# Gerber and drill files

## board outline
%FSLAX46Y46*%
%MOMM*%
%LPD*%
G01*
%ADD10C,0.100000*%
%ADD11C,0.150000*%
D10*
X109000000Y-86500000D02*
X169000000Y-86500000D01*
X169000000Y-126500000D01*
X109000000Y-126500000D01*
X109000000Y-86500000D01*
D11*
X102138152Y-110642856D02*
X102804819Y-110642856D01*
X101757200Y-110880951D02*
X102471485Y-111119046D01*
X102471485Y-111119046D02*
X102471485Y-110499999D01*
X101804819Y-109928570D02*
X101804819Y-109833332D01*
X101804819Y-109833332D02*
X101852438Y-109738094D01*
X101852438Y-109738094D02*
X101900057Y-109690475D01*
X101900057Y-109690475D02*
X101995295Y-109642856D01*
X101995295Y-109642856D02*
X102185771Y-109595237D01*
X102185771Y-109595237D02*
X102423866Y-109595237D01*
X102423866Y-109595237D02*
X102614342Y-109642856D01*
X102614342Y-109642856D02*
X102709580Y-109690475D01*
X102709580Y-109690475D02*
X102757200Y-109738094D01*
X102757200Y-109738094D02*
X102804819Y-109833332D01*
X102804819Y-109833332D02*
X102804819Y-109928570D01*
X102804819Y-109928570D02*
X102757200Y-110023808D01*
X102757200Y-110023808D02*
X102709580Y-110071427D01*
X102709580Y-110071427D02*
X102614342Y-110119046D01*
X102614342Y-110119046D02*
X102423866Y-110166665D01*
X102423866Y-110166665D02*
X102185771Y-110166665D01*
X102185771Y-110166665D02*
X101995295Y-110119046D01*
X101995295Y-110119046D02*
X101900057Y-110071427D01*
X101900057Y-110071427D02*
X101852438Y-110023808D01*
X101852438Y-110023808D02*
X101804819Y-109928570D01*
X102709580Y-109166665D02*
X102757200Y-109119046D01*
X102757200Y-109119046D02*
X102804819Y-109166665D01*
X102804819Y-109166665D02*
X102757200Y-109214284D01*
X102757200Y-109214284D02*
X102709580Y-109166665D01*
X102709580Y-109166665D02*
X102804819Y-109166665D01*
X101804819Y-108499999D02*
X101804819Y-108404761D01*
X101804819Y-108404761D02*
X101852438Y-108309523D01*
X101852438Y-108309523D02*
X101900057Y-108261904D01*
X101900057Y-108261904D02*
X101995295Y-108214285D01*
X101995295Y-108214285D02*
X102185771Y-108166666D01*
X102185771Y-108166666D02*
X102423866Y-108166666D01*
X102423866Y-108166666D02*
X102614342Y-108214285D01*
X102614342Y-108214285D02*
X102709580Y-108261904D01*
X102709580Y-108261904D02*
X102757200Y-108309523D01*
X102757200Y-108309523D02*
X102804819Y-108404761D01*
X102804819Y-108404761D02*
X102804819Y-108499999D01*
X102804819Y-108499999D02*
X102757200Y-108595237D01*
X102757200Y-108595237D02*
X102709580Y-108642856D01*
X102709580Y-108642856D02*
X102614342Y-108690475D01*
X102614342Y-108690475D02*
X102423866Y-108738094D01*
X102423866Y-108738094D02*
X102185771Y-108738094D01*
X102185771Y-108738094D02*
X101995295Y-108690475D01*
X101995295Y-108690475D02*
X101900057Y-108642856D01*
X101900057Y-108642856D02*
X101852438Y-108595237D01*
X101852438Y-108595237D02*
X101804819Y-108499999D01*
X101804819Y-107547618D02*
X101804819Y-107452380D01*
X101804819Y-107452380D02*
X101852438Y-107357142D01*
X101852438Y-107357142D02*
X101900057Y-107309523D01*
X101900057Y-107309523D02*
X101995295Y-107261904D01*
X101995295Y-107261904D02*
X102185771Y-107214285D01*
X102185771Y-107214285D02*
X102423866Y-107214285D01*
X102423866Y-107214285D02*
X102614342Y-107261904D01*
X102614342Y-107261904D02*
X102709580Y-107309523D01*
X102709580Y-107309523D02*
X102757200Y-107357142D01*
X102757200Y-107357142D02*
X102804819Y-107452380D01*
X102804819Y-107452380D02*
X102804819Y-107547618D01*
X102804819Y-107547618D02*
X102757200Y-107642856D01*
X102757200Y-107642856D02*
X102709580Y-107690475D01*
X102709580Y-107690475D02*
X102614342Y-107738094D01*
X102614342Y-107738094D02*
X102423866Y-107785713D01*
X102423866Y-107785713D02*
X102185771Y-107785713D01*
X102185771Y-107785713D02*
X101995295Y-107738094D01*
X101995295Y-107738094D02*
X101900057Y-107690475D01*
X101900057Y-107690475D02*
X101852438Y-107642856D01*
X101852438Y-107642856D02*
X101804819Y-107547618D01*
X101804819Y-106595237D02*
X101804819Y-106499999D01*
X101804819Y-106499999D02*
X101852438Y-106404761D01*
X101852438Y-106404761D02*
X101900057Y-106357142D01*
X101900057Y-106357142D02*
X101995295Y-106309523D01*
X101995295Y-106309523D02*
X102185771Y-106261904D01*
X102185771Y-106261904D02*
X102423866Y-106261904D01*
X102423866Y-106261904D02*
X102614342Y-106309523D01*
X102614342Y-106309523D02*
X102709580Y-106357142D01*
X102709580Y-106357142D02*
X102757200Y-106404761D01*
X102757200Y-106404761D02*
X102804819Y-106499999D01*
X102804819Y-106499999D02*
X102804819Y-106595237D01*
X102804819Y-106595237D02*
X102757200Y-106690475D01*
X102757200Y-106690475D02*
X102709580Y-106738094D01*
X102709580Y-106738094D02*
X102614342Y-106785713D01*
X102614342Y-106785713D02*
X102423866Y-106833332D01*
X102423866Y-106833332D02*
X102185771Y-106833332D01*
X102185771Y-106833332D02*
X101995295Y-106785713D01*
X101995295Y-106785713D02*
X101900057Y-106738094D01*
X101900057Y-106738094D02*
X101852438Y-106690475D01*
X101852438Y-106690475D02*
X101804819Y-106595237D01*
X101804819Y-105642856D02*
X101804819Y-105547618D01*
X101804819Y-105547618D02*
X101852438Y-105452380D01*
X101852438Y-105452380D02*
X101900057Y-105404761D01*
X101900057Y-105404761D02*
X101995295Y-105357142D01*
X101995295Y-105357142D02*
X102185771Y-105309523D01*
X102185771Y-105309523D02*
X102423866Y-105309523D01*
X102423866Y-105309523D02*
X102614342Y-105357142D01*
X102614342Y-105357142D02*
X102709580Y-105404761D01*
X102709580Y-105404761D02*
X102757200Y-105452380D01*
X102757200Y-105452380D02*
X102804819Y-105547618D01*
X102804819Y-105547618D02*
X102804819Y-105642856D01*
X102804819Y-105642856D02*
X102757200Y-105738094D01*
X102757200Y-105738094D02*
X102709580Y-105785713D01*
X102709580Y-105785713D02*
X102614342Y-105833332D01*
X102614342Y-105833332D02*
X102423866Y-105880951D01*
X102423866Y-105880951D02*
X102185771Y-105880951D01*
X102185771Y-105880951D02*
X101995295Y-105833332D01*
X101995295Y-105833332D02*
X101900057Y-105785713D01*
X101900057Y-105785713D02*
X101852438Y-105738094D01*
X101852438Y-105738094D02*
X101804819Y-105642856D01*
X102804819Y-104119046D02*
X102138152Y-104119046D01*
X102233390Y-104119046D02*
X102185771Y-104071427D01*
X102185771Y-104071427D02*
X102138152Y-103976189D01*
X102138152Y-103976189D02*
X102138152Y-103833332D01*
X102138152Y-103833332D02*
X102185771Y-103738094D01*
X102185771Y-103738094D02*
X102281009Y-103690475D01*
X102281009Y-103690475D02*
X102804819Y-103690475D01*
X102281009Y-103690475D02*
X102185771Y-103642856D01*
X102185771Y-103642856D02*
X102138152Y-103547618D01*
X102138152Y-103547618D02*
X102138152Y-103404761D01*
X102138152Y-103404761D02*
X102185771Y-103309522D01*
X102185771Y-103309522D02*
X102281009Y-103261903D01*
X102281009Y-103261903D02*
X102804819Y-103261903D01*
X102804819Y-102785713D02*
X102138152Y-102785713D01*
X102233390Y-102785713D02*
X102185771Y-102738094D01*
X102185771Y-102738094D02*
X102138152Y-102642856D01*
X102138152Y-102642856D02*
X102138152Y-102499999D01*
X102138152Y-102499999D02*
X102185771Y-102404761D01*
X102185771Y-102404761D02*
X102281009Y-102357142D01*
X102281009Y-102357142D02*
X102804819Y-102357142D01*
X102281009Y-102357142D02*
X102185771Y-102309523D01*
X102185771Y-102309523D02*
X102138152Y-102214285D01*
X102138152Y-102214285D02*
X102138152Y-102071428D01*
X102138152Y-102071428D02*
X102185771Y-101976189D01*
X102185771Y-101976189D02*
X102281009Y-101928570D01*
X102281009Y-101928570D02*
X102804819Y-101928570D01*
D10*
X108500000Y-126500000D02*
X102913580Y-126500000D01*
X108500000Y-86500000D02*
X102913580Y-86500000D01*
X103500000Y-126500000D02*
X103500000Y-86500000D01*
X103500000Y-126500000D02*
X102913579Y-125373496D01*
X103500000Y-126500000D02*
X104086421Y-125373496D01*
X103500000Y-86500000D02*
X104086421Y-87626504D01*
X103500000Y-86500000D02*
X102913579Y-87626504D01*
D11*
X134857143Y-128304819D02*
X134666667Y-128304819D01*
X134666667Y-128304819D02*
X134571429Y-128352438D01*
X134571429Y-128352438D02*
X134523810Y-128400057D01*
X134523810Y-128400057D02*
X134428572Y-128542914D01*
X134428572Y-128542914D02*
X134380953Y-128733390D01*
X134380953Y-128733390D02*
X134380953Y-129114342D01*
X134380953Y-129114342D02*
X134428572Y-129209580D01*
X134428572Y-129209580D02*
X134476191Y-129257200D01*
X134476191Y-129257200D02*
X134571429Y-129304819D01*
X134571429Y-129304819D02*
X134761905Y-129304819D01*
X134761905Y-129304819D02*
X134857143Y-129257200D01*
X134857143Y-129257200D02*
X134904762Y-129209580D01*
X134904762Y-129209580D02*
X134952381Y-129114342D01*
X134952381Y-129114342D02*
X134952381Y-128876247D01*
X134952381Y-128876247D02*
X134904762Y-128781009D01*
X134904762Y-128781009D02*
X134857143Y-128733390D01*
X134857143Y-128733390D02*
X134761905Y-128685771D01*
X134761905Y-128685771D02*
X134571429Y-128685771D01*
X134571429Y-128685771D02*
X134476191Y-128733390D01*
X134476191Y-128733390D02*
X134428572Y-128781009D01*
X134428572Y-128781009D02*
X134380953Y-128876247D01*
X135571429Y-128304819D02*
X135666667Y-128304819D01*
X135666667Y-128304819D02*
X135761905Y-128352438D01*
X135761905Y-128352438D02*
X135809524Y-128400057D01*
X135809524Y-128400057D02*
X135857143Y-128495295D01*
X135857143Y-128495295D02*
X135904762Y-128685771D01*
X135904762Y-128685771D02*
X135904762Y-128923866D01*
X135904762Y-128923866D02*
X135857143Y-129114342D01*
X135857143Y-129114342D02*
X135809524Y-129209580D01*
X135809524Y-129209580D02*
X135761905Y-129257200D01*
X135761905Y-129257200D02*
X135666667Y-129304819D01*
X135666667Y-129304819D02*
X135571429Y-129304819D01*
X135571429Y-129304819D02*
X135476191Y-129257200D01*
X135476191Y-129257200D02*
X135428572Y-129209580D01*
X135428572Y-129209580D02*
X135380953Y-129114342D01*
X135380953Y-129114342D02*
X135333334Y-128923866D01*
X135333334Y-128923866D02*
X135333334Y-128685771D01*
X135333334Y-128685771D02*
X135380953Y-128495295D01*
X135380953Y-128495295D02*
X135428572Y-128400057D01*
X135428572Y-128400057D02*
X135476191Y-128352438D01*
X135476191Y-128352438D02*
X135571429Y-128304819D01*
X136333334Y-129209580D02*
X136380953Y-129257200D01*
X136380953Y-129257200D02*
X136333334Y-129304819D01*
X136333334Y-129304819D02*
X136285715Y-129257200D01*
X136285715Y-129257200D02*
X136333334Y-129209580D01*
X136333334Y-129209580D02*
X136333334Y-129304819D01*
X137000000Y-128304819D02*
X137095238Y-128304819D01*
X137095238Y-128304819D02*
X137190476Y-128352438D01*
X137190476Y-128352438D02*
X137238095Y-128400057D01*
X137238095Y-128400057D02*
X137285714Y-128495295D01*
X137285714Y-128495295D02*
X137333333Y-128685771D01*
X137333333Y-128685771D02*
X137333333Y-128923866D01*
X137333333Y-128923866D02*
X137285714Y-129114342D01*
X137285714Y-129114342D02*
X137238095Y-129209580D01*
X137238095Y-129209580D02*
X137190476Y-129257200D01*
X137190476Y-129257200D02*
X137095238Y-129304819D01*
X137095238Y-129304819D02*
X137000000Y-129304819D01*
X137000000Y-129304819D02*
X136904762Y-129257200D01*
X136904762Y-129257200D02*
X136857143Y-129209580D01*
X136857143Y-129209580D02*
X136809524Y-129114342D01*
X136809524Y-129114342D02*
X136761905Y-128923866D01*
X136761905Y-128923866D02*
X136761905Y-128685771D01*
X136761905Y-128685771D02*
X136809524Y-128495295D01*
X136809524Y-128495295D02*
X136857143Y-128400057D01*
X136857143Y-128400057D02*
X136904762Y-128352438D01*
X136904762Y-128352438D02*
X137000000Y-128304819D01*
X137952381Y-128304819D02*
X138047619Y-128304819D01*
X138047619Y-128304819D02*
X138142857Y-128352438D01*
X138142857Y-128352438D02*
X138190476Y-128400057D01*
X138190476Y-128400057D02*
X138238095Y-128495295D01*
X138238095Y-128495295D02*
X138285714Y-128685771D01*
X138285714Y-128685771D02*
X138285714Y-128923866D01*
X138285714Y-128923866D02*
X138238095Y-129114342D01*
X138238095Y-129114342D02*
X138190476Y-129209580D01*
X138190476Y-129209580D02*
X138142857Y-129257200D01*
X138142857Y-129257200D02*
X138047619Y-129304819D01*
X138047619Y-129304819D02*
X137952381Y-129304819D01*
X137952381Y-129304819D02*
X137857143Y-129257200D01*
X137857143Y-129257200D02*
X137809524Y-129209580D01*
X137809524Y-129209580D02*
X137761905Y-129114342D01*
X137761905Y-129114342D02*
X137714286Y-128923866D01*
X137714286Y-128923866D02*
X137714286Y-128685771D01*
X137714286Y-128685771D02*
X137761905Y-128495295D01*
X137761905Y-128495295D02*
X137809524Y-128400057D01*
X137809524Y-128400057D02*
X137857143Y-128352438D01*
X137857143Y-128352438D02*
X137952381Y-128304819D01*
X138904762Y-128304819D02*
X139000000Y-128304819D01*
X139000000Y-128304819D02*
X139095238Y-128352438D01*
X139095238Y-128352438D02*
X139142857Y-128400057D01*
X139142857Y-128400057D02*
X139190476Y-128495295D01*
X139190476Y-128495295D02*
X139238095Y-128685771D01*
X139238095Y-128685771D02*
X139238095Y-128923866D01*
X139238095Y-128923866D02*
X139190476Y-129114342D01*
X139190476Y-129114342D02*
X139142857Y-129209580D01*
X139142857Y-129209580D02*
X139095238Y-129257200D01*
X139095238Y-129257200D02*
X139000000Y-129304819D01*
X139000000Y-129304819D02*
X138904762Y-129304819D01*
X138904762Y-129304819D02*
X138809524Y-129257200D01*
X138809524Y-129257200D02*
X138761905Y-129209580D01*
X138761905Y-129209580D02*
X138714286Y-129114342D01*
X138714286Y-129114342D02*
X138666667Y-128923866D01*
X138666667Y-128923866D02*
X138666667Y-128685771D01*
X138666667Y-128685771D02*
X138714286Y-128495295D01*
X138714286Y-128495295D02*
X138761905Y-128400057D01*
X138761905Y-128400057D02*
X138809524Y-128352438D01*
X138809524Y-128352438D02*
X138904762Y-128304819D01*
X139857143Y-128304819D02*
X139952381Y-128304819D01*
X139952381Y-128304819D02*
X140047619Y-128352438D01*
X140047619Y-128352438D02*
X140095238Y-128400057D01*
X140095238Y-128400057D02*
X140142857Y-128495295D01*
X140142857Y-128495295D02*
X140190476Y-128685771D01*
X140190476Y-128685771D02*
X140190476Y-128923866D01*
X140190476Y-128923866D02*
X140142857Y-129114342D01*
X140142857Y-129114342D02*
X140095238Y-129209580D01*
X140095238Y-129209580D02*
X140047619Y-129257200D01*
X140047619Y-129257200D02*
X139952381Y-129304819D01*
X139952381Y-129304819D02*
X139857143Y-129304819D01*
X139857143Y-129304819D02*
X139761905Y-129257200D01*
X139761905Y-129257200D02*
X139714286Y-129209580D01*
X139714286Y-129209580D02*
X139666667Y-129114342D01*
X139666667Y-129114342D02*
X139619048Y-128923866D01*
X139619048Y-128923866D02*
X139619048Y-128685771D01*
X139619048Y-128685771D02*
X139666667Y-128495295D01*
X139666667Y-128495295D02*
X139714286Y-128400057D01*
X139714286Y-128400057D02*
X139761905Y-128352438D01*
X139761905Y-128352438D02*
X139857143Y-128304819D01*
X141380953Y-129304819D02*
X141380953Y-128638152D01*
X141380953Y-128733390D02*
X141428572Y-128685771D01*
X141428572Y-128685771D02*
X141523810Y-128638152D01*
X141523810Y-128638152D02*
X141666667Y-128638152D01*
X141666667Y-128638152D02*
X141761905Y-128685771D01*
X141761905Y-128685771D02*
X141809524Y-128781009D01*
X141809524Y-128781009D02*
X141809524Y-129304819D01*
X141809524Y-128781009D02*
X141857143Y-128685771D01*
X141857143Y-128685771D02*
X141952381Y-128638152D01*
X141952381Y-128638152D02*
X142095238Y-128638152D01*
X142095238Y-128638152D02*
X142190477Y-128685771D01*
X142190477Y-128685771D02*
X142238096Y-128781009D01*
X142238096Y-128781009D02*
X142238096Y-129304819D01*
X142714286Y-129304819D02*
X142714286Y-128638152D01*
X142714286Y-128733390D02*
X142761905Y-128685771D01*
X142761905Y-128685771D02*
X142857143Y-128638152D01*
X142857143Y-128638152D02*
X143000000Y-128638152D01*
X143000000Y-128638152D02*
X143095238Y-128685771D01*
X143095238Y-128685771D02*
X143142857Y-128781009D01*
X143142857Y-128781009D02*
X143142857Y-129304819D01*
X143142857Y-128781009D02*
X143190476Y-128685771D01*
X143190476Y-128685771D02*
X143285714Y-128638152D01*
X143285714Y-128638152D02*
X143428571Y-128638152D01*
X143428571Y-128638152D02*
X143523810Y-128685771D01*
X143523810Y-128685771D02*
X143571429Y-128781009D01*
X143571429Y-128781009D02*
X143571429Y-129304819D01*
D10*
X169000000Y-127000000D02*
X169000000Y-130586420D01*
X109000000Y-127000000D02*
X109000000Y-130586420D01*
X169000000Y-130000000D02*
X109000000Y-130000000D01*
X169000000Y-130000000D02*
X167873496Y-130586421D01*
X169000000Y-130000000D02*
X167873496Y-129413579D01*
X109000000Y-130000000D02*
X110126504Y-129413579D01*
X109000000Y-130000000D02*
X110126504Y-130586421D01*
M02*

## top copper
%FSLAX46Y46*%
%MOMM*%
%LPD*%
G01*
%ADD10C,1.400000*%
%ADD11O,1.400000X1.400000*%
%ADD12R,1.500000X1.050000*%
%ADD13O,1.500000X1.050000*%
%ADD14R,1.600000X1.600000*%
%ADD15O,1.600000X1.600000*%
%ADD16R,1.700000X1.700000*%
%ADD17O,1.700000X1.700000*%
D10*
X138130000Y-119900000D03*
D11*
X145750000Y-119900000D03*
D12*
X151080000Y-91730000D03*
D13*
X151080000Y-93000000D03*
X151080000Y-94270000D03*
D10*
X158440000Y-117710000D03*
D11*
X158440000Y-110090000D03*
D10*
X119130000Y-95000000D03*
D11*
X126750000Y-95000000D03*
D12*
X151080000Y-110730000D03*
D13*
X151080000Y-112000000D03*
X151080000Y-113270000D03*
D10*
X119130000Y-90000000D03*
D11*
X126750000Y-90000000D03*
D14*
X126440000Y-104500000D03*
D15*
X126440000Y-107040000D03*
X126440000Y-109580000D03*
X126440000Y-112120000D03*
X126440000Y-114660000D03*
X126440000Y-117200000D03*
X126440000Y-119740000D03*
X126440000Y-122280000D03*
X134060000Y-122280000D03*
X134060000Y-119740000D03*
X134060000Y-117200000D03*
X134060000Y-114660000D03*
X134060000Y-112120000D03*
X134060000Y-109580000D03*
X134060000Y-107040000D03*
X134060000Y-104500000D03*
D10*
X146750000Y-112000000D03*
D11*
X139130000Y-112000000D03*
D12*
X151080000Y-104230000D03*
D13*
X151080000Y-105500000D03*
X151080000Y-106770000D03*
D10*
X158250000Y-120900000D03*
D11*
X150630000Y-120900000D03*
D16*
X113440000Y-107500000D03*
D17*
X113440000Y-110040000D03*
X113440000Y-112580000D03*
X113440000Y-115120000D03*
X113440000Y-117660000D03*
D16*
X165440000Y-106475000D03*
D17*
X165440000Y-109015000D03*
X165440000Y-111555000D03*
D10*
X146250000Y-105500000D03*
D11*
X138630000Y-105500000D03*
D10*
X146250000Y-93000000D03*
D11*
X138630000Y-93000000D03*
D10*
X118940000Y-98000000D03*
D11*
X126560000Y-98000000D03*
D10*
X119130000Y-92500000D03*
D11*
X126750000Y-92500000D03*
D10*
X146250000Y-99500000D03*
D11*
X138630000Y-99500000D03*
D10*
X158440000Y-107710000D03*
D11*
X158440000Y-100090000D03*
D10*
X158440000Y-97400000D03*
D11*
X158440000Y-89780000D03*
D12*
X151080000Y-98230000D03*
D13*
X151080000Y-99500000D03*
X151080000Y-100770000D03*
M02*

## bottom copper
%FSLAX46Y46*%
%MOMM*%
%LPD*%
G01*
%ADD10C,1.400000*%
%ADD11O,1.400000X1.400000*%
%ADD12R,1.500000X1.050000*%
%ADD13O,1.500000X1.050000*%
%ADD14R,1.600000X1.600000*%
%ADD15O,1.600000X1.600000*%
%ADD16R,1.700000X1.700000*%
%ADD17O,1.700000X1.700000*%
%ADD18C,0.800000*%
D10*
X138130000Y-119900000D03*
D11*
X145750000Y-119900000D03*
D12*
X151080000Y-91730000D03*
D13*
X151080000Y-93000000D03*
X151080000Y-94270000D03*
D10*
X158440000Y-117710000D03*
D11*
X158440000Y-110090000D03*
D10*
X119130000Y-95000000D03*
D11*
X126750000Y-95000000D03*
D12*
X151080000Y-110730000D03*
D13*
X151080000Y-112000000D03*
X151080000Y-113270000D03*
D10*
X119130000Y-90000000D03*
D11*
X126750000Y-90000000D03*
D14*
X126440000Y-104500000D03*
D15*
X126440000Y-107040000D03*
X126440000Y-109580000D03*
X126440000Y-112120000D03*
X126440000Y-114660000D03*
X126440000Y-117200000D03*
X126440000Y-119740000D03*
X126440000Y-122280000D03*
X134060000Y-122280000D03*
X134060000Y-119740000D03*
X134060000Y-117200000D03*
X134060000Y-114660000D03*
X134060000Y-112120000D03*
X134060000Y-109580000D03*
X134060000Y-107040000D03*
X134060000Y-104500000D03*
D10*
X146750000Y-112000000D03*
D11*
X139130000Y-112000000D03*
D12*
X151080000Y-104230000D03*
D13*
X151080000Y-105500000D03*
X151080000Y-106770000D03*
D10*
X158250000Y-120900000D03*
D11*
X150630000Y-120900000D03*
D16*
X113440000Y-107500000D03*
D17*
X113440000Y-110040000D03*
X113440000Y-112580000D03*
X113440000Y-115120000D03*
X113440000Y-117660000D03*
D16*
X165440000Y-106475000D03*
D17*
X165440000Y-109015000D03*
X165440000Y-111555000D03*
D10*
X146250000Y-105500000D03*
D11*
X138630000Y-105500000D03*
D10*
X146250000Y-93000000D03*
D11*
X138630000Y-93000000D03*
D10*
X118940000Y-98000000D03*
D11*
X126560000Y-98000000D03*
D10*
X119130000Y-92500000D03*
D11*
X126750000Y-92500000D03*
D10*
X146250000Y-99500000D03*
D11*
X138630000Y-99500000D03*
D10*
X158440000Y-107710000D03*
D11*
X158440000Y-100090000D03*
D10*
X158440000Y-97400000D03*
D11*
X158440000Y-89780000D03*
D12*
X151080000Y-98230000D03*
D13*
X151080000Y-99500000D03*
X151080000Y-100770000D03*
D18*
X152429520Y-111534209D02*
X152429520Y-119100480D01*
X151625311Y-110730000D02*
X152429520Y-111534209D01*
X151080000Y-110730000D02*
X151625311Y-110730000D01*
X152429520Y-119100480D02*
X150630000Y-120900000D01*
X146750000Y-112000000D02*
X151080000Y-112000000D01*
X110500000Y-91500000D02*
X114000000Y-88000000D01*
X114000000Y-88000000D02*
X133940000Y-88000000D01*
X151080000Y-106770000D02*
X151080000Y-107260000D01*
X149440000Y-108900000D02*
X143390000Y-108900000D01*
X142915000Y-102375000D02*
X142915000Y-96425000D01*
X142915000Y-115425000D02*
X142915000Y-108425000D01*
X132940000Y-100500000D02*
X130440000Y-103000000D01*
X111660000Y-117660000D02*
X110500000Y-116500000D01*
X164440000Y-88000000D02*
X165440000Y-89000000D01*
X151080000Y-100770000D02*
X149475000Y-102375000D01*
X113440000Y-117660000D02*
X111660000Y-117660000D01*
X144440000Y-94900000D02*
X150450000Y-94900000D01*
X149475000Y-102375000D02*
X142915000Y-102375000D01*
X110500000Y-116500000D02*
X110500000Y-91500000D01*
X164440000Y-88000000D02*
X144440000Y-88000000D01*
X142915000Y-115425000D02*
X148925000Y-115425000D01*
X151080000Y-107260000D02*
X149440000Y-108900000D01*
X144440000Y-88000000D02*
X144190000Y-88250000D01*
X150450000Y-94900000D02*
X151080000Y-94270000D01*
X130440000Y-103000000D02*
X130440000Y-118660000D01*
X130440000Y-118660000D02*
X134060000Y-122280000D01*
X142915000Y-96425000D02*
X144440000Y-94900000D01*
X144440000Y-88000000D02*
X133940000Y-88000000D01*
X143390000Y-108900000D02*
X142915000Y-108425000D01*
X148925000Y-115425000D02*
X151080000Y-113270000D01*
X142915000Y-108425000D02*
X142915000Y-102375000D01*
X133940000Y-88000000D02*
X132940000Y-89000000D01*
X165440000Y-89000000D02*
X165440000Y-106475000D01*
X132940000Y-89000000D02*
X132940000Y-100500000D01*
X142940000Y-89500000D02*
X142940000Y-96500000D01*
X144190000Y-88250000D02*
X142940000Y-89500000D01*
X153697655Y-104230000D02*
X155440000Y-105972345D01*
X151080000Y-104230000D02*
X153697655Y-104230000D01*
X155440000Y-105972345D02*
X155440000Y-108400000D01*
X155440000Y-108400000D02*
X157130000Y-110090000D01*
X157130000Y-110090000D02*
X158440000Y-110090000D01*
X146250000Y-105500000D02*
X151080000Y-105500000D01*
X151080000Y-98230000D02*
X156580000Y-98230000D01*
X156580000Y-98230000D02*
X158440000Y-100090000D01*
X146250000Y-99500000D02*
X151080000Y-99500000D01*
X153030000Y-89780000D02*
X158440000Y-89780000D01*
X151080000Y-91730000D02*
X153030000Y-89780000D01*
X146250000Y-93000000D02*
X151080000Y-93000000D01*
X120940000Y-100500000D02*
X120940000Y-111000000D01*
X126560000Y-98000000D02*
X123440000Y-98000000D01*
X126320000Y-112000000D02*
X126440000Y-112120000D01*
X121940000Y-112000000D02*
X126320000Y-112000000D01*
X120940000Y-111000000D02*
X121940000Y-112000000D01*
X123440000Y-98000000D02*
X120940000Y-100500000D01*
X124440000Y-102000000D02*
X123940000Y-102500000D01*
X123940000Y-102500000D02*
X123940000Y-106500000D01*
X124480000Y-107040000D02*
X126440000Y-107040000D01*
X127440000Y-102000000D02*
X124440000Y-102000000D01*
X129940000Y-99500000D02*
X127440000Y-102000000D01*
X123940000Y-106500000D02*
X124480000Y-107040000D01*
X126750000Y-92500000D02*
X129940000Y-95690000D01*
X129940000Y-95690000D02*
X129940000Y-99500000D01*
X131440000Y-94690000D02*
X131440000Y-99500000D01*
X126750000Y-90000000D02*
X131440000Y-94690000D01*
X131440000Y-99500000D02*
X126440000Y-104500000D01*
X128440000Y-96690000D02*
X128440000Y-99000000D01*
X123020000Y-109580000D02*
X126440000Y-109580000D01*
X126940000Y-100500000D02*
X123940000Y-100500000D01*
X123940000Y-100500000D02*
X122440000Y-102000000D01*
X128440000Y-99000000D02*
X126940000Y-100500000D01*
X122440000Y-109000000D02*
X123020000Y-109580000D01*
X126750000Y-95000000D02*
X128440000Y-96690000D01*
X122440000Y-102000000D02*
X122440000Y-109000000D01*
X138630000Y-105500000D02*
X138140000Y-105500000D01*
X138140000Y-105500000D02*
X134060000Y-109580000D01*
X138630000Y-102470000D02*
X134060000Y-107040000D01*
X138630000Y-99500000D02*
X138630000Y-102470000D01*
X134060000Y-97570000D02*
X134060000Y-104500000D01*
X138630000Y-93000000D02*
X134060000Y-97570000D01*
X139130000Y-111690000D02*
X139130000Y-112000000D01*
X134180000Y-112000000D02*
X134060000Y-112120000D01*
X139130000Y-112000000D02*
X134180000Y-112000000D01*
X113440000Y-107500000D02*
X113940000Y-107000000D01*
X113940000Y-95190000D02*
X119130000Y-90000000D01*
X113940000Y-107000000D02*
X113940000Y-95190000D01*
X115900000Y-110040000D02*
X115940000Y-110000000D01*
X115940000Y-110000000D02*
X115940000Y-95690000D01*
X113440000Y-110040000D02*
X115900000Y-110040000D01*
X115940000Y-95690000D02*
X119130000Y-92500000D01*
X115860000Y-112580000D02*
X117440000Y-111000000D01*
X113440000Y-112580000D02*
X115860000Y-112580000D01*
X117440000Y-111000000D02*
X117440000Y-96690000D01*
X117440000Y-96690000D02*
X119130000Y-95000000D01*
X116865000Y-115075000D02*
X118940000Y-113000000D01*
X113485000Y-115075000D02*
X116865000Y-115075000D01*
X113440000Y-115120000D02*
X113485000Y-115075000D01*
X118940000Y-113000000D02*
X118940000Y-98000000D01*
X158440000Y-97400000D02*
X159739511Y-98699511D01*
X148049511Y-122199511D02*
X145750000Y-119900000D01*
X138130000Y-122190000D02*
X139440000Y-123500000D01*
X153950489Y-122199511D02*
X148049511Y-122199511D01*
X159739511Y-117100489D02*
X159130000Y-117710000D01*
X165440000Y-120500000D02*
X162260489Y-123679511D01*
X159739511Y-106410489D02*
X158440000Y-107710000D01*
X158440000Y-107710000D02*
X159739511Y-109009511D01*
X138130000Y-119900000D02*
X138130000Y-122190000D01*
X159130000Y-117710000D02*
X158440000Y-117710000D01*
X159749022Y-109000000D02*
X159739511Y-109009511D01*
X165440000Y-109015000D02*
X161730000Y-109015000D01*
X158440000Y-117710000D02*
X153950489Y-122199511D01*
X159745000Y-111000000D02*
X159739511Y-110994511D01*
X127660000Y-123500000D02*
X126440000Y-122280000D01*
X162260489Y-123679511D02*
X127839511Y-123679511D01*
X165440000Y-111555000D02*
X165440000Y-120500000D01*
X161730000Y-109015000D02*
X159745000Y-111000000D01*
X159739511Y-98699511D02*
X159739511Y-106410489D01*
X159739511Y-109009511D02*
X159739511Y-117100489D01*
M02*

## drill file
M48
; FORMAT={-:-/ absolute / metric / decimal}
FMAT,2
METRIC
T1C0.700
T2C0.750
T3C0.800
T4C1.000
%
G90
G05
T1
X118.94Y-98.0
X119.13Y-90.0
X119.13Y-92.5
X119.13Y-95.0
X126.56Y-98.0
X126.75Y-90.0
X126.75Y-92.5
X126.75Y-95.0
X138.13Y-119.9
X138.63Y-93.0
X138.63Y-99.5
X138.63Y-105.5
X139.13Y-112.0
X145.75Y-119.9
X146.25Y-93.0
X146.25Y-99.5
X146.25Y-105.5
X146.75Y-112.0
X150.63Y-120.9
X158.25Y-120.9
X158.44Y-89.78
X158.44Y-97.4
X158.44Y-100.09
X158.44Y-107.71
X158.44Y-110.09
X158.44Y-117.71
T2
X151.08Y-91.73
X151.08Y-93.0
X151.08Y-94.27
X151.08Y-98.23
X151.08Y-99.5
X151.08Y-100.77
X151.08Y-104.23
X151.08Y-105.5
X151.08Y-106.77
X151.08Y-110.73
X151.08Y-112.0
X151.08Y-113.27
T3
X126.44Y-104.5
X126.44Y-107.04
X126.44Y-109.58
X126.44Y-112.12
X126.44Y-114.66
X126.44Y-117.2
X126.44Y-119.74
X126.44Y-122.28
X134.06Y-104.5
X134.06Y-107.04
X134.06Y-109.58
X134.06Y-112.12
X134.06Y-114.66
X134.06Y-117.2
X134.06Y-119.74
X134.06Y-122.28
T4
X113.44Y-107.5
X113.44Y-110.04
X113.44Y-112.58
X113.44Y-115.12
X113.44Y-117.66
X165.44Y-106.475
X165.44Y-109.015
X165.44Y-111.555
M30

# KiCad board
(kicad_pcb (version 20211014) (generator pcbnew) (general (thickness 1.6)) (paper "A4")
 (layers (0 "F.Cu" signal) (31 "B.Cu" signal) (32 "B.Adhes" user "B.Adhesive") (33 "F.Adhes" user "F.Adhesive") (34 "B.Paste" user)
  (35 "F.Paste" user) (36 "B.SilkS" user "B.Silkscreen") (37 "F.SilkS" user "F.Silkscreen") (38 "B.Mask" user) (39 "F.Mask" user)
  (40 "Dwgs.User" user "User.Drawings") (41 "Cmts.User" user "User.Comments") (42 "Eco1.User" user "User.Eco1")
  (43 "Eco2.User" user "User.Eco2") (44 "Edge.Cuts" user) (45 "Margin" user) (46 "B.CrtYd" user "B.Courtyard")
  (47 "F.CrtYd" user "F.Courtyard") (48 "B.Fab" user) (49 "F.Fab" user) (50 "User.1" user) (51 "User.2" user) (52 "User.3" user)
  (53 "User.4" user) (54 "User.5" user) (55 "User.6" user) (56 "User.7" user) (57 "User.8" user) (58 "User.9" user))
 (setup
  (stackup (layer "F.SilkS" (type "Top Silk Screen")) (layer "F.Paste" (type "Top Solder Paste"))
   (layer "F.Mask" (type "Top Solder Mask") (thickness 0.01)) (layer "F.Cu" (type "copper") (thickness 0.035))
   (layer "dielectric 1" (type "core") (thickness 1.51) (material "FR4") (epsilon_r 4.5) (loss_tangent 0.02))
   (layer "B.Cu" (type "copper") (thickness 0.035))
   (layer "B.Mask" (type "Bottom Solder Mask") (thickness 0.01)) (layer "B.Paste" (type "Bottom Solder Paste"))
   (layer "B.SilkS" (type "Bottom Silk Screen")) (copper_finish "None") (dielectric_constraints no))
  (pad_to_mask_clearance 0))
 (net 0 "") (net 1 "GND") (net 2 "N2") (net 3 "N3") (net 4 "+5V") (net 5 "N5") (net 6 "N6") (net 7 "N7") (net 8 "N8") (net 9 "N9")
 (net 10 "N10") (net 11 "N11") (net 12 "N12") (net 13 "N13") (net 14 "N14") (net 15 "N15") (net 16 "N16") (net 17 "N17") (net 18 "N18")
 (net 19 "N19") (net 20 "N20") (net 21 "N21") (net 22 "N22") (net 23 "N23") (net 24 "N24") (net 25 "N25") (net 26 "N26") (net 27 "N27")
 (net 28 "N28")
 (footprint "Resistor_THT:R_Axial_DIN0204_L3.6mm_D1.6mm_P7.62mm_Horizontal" (layer "F.Cu") (at 138.13 119.9)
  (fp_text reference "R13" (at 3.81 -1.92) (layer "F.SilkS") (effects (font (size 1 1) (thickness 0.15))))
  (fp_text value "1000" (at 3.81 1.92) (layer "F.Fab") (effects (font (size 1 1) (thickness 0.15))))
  (pad "1" thru_hole circle (at 0 0) (size 1.4 1.4) (drill 0.7) (layers *.Cu *.Mask) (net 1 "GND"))
  (pad "2" thru_hole oval (at 7.62 0) (size 1.4 1.4) (drill 0.7) (layers *.Cu *.Mask) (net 1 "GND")))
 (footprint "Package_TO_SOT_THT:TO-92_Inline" (layer "F.Cu") (at 151.08 91.73 -90)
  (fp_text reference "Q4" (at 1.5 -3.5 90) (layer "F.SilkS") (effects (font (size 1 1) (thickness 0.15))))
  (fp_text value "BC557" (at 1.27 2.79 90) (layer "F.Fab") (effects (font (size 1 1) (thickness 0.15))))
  (pad "1" thru_hole rect (at 0 0 270) (size 1.05 1.5) (drill 0.75) (layers *.Cu *.Mask) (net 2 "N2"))
  (pad "2" thru_hole oval (at 1.27 0 270) (size 1.05 1.5) (drill 0.75) (layers *.Cu *.Mask) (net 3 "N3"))
  (pad "3" thru_hole oval (at 2.54 0 270) (size 1.05 1.5) (drill 0.75) (layers *.Cu *.Mask) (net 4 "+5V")))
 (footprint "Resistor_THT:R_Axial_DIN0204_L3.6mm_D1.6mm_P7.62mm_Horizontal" (layer "F.Cu") (at 158.44 117.71 90)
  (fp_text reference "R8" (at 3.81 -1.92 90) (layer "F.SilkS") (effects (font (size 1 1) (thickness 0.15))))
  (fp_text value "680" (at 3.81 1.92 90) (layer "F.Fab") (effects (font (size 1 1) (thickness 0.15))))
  (pad "1" thru_hole circle (at 0 0 90) (size 1.4 1.4) (drill 0.7) (layers *.Cu *.Mask) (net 1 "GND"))
  (pad "2" thru_hole oval (at 7.62 0 90) (size 1.4 1.4) (drill 0.7) (layers *.Cu *.Mask) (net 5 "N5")))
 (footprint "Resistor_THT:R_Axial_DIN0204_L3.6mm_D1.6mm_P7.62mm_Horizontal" (layer "F.Cu") (at 119.13 95)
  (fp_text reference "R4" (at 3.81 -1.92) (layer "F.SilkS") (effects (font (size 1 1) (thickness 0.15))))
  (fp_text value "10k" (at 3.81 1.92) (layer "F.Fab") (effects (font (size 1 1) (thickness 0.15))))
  (pad "1" thru_hole circle (at 0 0) (size 1.4 1.4) (drill 0.7) (layers *.Cu *.Mask) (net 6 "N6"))
  (pad "2" thru_hole oval (at 7.62 0) (size 1.4 1.4) (drill 0.7) (layers *.Cu *.Mask) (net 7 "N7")))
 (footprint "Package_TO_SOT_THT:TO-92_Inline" (layer "F.Cu") (at 151.08 110.73 -90)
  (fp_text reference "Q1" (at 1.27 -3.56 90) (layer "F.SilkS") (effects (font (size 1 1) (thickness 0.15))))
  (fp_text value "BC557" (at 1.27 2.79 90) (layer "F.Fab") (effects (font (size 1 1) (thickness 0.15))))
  (pad "1" thru_hole rect (at 0 0 270) (size 1.05 1.5) (drill 0.75) (layers *.Cu *.Mask) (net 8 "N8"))
  (pad "2" thru_hole oval (at 1.27 0 270) (size 1.05 1.5) (drill 0.75) (layers *.Cu *.Mask) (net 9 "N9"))
  (pad "3" thru_hole oval (at 2.54 0 270) (size 1.05 1.5) (drill 0.75) (layers *.Cu *.Mask) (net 4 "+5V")))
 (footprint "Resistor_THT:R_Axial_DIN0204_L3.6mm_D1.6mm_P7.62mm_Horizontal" (layer "F.Cu") (at 119.13 90)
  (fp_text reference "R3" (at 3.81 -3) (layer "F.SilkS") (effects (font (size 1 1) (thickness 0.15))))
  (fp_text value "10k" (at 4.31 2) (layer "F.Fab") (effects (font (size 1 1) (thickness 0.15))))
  (pad "1" thru_hole circle (at 0 0) (size 1.4 1.4) (drill 0.7) (layers *.Cu *.Mask) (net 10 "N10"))
  (pad "2" thru_hole oval (at 7.62 0) (size 1.4 1.4) (drill 0.7) (layers *.Cu *.Mask) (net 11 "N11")))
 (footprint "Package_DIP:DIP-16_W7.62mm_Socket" (layer "F.Cu") (at 126.44 104.5)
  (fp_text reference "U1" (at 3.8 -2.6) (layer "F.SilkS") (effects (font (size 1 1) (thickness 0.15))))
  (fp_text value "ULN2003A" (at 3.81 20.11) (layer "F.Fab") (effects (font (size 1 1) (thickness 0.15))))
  (pad "1" thru_hole rect (at 0 0) (size 1.6 1.6) (drill 0.8) (layers *.Cu *.Mask) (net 11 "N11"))
  (pad "2" thru_hole oval (at 0 2.54) (size 1.6 1.6) (drill 0.8) (layers *.Cu *.Mask) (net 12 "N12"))
  (pad "3" thru_hole oval (at 0 5.08) (size 1.6 1.6) (drill 0.8) (layers *.Cu *.Mask) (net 7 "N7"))
  (pad "4" thru_hole oval (at 0 7.62) (size 1.6 1.6) (drill 0.8) (layers *.Cu *.Mask) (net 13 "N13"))
  (pad "5" thru_hole oval (at 0 10.16) (size 1.6 1.6) (drill 0.8) (layers *.Cu *.Mask) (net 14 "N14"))
  (pad "6" thru_hole oval (at 0 12.7) (size 1.6 1.6) (drill 0.8) (layers *.Cu *.Mask) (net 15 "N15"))
  (pad "7" thru_hole oval (at 0 15.24) (size 1.6 1.6) (drill 0.8) (layers *.Cu *.Mask) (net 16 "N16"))
  (pad "8" thru_hole oval (at 0 17.78) (size 1.6 1.6) (drill 0.8) (layers *.Cu *.Mask) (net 1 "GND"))
  (pad "9" thru_hole oval (at 7.62 17.78) (size 1.6 1.6) (drill 0.8) (layers *.Cu *.Mask) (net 4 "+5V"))
  (pad "10" thru_hole oval (at 7.62 15.24) (size 1.6 1.6) (drill 0.8) (layers *.Cu *.Mask) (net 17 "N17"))
  (pad "11" thru_hole oval (at 7.62 12.7) (size 1.6 1.6) (drill 0.8) (layers *.Cu *.Mask) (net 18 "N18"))
  (pad "12" thru_hole oval (at 7.62 10.16) (size 1.6 1.6) (drill 0.8) (layers *.Cu *.Mask) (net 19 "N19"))
  (pad "13" thru_hole oval (at 7.62 7.62) (size 1.6 1.6) (drill 0.8) (layers *.Cu *.Mask) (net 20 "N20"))
  (pad "14" thru_hole oval (at 7.62 5.08) (size 1.6 1.6) (drill 0.8) (layers *.Cu *.Mask) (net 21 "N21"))
  (pad "15" thru_hole oval (at 7.62 2.54) (size 1.6 1.6) (drill 0.8) (layers *.Cu *.Mask) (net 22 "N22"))
  (pad "16" thru_hole oval (at 7.62 0) (size 1.6 1.6) (drill 0.8) (layers *.Cu *.Mask) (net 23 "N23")))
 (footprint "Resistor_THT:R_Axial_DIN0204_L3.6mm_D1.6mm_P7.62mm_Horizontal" (layer "F.Cu") (at 146.75 112 180)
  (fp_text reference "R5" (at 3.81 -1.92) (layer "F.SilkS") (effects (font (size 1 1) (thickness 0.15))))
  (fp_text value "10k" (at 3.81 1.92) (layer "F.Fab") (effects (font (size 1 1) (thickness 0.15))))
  (pad "1" thru_hole circle (at 0 0 180) (size 1.4 1.4) (drill 0.7) (layers *.Cu *.Mask) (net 9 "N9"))
  (pad "2" thru_hole oval (at 7.62 0 180) (size 1.4 1.4) (drill 0.7) (layers *.Cu *.Mask) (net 20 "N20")))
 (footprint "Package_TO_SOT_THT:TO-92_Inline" (layer "F.Cu") (at 151.08 104.23 -90)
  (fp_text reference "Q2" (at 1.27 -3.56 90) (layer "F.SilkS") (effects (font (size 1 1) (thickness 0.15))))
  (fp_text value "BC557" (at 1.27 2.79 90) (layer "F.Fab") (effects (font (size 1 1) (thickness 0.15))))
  (pad "1" thru_hole rect (at 0 0 270) (size 1.05 1.5) (drill 0.75) (layers *.Cu *.Mask) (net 5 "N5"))
  (pad "2" thru_hole oval (at 1.27 0 270) (size 1.05 1.5) (drill 0.75) (layers *.Cu *.Mask) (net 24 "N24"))
  (pad "3" thru_hole oval (at 2.54 0 270) (size 1.05 1.5) (drill 0.75) (layers *.Cu *.Mask) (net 4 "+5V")))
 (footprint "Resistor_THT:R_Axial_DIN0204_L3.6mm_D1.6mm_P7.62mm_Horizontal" (layer "F.Cu") (at 158.25 120.9 180)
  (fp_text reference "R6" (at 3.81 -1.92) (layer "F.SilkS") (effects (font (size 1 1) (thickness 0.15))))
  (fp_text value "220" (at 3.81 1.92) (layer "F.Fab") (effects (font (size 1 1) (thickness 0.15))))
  (pad "1" thru_hole circle (at 0 0 180) (size 1.4 1.4) (drill 0.7) (layers *.Cu *.Mask) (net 1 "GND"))
  (pad "2" thru_hole oval (at 7.62 0 180) (size 1.4 1.4) (drill 0.7) (layers *.Cu *.Mask) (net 8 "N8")))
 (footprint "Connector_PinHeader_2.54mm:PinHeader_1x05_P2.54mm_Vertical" (layer "F.Cu") (at 113.44 107.5)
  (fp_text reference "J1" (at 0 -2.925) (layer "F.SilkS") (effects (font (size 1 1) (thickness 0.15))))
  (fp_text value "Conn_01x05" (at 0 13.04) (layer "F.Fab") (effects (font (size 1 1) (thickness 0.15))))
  (pad "1" thru_hole rect (at 0 0) (size 1.7 1.7) (drill 1) (layers *.Cu *.Mask) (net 10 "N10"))
  (pad "2" thru_hole oval (at 0 2.54) (size 1.7 1.7) (drill 1) (layers *.Cu *.Mask) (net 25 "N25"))
  (pad "3" thru_hole oval (at 0 5.08) (size 1.7 1.7) (drill 1) (layers *.Cu *.Mask) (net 6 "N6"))
  (pad "4" thru_hole oval (at 0 7.62) (size 1.7 1.7) (drill 1) (layers *.Cu *.Mask) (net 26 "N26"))
  (pad "5" thru_hole oval (at 0 10.16) (size 1.7 1.7) (drill 1) (layers *.Cu *.Mask) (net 4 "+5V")))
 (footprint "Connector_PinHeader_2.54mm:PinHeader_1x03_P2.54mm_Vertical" (layer "F.Cu") (at 165.44 106.475)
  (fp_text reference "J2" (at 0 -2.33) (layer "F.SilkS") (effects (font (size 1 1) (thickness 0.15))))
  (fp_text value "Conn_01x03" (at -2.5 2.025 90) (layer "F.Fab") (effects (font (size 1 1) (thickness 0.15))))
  (pad "1" thru_hole rect (at 0 0) (size 1.7 1.7) (drill 1) (layers *.Cu *.Mask) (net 4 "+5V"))
  (pad "2" thru_hole oval (at 0 2.54) (size 1.7 1.7) (drill 1) (layers *.Cu *.Mask) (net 1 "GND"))
  (pad "3" thru_hole oval (at 0 5.08) (size 1.7 1.7) (drill 1) (layers *.Cu *.Mask) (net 1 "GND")))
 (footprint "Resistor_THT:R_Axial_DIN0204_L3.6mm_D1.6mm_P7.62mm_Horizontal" (layer "F.Cu") (at 146.25 105.5 180)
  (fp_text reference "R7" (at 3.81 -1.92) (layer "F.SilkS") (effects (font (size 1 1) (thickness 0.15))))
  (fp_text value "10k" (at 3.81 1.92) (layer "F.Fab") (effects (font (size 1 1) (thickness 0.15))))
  (pad "1" thru_hole circle (at 0 0 180) (size 1.4 1.4) (drill 0.7) (layers *.Cu *.Mask) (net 24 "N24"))
  (pad "2" thru_hole oval (at 7.62 0 180) (size 1.4 1.4) (drill 0.7) (layers *.Cu *.Mask) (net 21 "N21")))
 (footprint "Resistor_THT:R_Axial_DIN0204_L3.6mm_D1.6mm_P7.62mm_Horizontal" (layer "F.Cu") (at 146.25 93 180)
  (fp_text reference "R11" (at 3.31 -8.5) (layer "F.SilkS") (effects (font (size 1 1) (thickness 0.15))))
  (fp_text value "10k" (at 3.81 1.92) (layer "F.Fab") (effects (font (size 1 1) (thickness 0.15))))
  (pad "1" thru_hole circle (at 0 0 180) (size 1.4 1.4) (drill 0.7) (layers *.Cu *.Mask) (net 3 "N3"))
  (pad "2" thru_hole oval (at 7.62 0 180) (size 1.4 1.4) (drill 0.7) (layers *.Cu *.Mask) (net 23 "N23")))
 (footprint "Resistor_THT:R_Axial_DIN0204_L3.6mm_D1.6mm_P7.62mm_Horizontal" (layer "F.Cu") (at 118.94 98)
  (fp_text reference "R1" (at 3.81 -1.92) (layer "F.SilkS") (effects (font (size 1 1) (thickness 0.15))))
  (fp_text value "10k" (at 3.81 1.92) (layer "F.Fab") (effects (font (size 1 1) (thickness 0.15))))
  (pad "1" thru_hole circle (at 0 0) (size 1.4 1.4) (drill 0.7) (layers *.Cu *.Mask) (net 26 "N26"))
  (pad "2" thru_hole oval (at 7.62 0) (size 1.4 1.4) (drill 0.7) (layers *.Cu *.Mask) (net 13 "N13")))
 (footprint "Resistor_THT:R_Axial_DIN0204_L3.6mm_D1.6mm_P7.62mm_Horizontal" (layer "F.Cu") (at 119.13 92.5)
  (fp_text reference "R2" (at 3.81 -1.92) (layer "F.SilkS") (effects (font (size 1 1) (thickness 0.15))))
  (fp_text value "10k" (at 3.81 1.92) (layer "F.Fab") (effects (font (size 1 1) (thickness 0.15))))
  (pad "1" thru_hole circle (at 0 0) (size 1.4 1.4) (drill 0.7) (layers *.Cu *.Mask) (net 25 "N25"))
  (pad "2" thru_hole oval (at 7.62 0) (size 1.4 1.4) (drill 0.7) (layers *.Cu *.Mask) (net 12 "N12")))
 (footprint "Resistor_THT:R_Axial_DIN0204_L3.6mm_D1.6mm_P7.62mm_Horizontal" (layer "F.Cu") (at 146.25 99.5 180)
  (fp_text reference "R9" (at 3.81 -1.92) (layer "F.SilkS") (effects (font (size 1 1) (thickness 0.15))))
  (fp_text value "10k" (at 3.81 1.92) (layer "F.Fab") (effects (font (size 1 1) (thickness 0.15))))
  (pad "1" thru_hole circle (at 0 0 180) (size 1.4 1.4) (drill 0.7) (layers *.Cu *.Mask) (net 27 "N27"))
  (pad "2" thru_hole oval (at 7.62 0 180) (size 1.4 1.4) (drill 0.7) (layers *.Cu *.Mask) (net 22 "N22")))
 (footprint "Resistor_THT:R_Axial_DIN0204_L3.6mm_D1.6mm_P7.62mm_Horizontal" (layer "F.Cu") (at 158.44 107.71 90)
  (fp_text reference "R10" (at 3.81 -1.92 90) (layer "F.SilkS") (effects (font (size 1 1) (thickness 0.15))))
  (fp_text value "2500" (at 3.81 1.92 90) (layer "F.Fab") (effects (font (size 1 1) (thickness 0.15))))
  (pad "1" thru_hole circle (at 0 0 90) (size 1.4 1.4) (drill 0.7) (layers *.Cu *.Mask) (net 1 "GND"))
  (pad "2" thru_hole oval (at 7.62 0 90) (size 1.4 1.4) (drill 0.7) (layers *.Cu *.Mask) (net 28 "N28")))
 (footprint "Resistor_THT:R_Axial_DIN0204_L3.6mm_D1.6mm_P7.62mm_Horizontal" (layer "F.Cu") (at 158.44 97.4 90)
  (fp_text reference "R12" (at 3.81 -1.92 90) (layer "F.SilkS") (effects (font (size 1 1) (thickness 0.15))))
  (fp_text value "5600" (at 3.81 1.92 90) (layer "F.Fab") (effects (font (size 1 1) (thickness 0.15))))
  (pad "1" thru_hole circle (at 0 0 90) (size 1.4 1.4) (drill 0.7) (layers *.Cu *.Mask) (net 1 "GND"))
  (pad "2" thru_hole oval (at 7.62 0 90) (size 1.4 1.4) (drill 0.7) (layers *.Cu *.Mask) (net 2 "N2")))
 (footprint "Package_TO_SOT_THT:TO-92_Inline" (layer "F.Cu") (at 151.08 98.23 -90)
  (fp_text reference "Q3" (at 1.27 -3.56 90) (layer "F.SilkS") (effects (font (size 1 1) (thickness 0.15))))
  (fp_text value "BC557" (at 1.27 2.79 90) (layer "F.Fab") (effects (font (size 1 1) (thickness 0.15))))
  (pad "1" thru_hole rect (at 0 0 270) (size 1.05 1.5) (drill 0.75) (layers *.Cu *.Mask) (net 28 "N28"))
  (pad "2" thru_hole oval (at 1.27 0 270) (size 1.05 1.5) (drill 0.75) (layers *.Cu *.Mask) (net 27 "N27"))
  (pad "3" thru_hole oval (at 2.54 0 270) (size 1.05 1.5) (drill 0.75) (layers *.Cu *.Mask) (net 4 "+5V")))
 (gr_rect (start 169 126.5) (end 109 86.5) (layer "Edge.Cuts") (width 0.1) (fill none))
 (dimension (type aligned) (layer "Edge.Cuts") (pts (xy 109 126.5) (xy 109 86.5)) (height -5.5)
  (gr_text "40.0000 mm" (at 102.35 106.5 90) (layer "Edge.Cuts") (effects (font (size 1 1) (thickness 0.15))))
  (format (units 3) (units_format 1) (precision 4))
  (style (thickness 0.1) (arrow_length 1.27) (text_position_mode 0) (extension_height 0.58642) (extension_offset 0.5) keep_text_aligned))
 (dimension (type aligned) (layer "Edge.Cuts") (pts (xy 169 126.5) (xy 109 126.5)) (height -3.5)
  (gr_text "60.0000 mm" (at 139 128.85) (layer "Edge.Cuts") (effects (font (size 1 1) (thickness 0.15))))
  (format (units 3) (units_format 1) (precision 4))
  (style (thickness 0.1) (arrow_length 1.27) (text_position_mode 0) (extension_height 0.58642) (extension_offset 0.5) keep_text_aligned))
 (segment (start 152.42952 111.534209) (end 152.42952 119.10048) (width 0.8) (layer "B.Cu") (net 8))
 (segment (start 151.625311 110.73) (end 152.42952 111.534209) (width 0.8) (layer "B.Cu") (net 8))
 (segment (start 151.08 110.73) (end 151.625311 110.73) (width 0.8) (layer "B.Cu") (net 8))
 (segment (start 152.42952 119.10048) (end 150.63 120.9) (width 0.8) (layer "B.Cu") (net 8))
 (segment (start 146.75 112) (end 151.08 112) (width 0.8) (layer "B.Cu") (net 9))
 (segment (start 110.5 91.5) (end 114 88) (width 0.8) (layer "B.Cu") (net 4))
 (segment (start 114 88) (end 133.94 88) (width 0.8) (layer "B.Cu") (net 4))
 (segment (start 151.08 106.77) (end 151.08 107.26) (width 0.8) (layer "B.Cu") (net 4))
 (segment (start 149.44 108.9) (end 143.39 108.9) (width 0.8) (layer "B.Cu") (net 4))
 (segment (start 142.915 102.375) (end 142.915 96.425) (width 0.8) (layer "B.Cu") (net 4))
 (segment (start 142.915 115.425) (end 142.915 108.425) (width 0.8) (layer "B.Cu") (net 4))
 (segment (start 132.94 100.5) (end 130.44 103) (width 0.8) (layer "B.Cu") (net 4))
 (segment (start 111.66 117.66) (end 110.5 116.5) (width 0.8) (layer "B.Cu") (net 4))
 (segment (start 164.44 88) (end 165.44 89) (width 0.8) (layer "B.Cu") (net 4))
 (segment (start 151.08 100.77) (end 149.475 102.375) (width 0.8) (layer "B.Cu") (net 4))
 (segment (start 113.44 117.66) (end 111.66 117.66) (width 0.8) (layer "B.Cu") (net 4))
 (segment (start 144.44 94.9) (end 150.45 94.9) (width 0.8) (layer "B.Cu") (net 4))
 (segment (start 149.475 102.375) (end 142.915 102.375) (width 0.8) (layer "B.Cu") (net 4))
 (segment (start 110.5 116.5) (end 110.5 91.5) (width 0.8) (layer "B.Cu") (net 4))
 (segment (start 164.44 88) (end 144.44 88) (width 0.8) (layer "B.Cu") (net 4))
 (segment (start 142.915 115.425) (end 148.925 115.425) (width 0.8) (layer "B.Cu") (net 4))
 (segment (start 151.08 107.26) (end 149.44 108.9) (width 0.8) (layer "B.Cu") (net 4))
 (segment (start 144.44 88) (end 144.19 88.25) (width 0.8) (layer "B.Cu") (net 4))
 (segment (start 150.45 94.9) (end 151.08 94.27) (width 0.8) (layer "B.Cu") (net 4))
 (segment (start 130.44 103) (end 130.44 118.66) (width 0.8) (layer "B.Cu") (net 4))
 (segment (start 130.44 118.66) (end 134.06 122.28) (width 0.8) (layer "B.Cu") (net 4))
 (segment (start 142.915 96.425) (end 144.44 94.9) (width 0.8) (layer "B.Cu") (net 4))
 (segment (start 144.44 88) (end 133.94 88) (width 0.8) (layer "B.Cu") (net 4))
 (segment (start 143.39 108.9) (end 142.915 108.425) (width 0.8) (layer "B.Cu") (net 4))
 (segment (start 148.925 115.425) (end 151.08 113.27) (width 0.8) (layer "B.Cu") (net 4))
 (segment (start 142.915 108.425) (end 142.915 102.375) (width 0.8) (layer "B.Cu") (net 4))
 (segment (start 133.94 88) (end 132.94 89) (width 0.8) (layer "B.Cu") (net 4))
 (segment (start 165.44 89) (end 165.44 106.475) (width 0.8) (layer "B.Cu") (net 4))
 (segment (start 132.94 89) (end 132.94 100.5) (width 0.8) (layer "B.Cu") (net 4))
 (segment (start 142.94 89.5) (end 142.94 96.5) (width 0.8) (layer "B.Cu") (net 4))
 (segment (start 144.19 88.25) (end 142.94 89.5) (width 0.8) (layer "B.Cu") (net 4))
 (segment (start 153.697655 104.23) (end 155.44 105.972345) (width 0.8) (layer "B.Cu") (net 5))
 (segment (start 151.08 104.23) (end 153.697655 104.23) (width 0.8) (layer "B.Cu") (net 5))
 (segment (start 155.44 105.972345) (end 155.44 108.4) (width 0.8) (layer "B.Cu") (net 5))
 (segment (start 155.44 108.4) (end 157.13 110.09) (width 0.8) (layer "B.Cu") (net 5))
 (segment (start 157.13 110.09) (end 158.44 110.09) (width 0.8) (layer "B.Cu") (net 5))
 (segment (start 146.25 105.5) (end 151.08 105.5) (width 0.8) (layer "B.Cu") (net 24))
 (segment (start 151.08 98.23) (end 156.58 98.23) (width 0.8) (layer "B.Cu") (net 28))
 (segment (start 156.58 98.23) (end 158.44 100.09) (width 0.8) (layer "B.Cu") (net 28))
 (segment (start 146.25 99.5) (end 151.08 99.5) (width 0.8) (layer "B.Cu") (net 27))
 (segment (start 153.03 89.78) (end 158.44 89.78) (width 0.8) (layer "B.Cu") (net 2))
 (segment (start 151.08 91.73) (end 153.03 89.78) (width 0.8) (layer "B.Cu") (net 2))
 (segment (start 146.25 93) (end 151.08 93) (width 0.8) (layer "B.Cu") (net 3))
 (segment (start 120.94 100.5) (end 120.94 111) (width 0.8) (layer "B.Cu") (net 13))
 (segment (start 126.56 98) (end 123.44 98) (width 0.8) (layer "B.Cu") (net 13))
 (segment (start 126.32 112) (end 126.44 112.12) (width 0.8) (layer "B.Cu") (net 13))
 (segment (start 121.94 112) (end 126.32 112) (width 0.8) (layer "B.Cu") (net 13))
 (segment (start 120.94 111) (end 121.94 112) (width 0.8) (layer "B.Cu") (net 13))
 (segment (start 123.44 98) (end 120.94 100.5) (width 0.8) (layer "B.Cu") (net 13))
 (segment (start 124.44 102) (end 123.94 102.5) (width 0.8) (layer "B.Cu") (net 12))
 (segment (start 123.94 102.5) (end 123.94 106.5) (width 0.8) (layer "B.Cu") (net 12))
 (segment (start 124.48 107.04) (end 126.44 107.04) (width 0.8) (layer "B.Cu") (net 12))
 (segment (start 127.44 102) (end 124.44 102) (width 0.8) (layer "B.Cu") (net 12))
 (segment (start 129.94 99.5) (end 127.44 102) (width 0.8) (layer "B.Cu") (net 12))
 (segment (start 123.94 106.5) (end 124.48 107.04) (width 0.8) (layer "B.Cu") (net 12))
 (segment (start 126.75 92.5) (end 129.94 95.69) (width 0.8) (layer "B.Cu") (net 12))
 (segment (start 129.94 95.69) (end 129.94 99.5) (width 0.8) (layer "B.Cu") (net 12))
 (segment (start 131.44 94.69) (end 131.44 99.5) (width 0.8) (layer "B.Cu") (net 11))
 (segment (start 126.75 90) (end 131.44 94.69) (width 0.8) (layer "B.Cu") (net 11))
 (segment (start 131.44 99.5) (end 126.44 104.5) (width 0.8) (layer "B.Cu") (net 11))
 (segment (start 128.44 96.69) (end 128.44 99) (width 0.8) (layer "B.Cu") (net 7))
 (segment (start 123.02 109.58) (end 126.44 109.58) (width 0.8) (layer "B.Cu") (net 7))
 (segment (start 126.94 100.5) (end 123.94 100.5) (width 0.8) (layer "B.Cu") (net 7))
 (segment (start 123.94 100.5) (end 122.44 102) (width 0.8) (layer "B.Cu") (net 7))
 (segment (start 128.44 99) (end 126.94 100.5) (width 0.8) (layer "B.Cu") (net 7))
 (segment (start 122.44 109) (end 123.02 109.58) (width 0.8) (layer "B.Cu") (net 7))
 (segment (start 126.75 95) (end 128.44 96.69) (width 0.8) (layer "B.Cu") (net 7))
 (segment (start 122.44 102) (end 122.44 109) (width 0.8) (layer "B.Cu") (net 7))
 (segment (start 138.63 105.5) (end 138.14 105.5) (width 0.8) (layer "B.Cu") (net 21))
 (segment (start 138.14 105.5) (end 134.06 109.58) (width 0.8) (layer "B.Cu") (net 21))
 (segment (start 138.63 102.47) (end 134.06 107.04) (width 0.8) (layer "B.Cu") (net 22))
 (segment (start 138.63 99.5) (end 138.63 102.47) (width 0.8) (layer "B.Cu") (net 22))
 (segment (start 134.06 97.57) (end 134.06 104.5) (width 0.8) (layer "B.Cu") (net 23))
 (segment (start 138.63 93) (end 134.06 97.57) (width 0.8) (layer "B.Cu") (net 23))
 (segment (start 139.13 111.69) (end 139.13 112) (width 0.8) (layer "B.Cu") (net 20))
 (segment (start 134.18 112) (end 134.06 112.12) (width 0.8) (layer "B.Cu") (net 20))
 (segment (start 139.13 112) (end 134.18 112) (width 0.8) (layer "B.Cu") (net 20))
 (segment (start 113.44 107.5) (end 113.94 107) (width 0.8) (layer "B.Cu") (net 10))
 (segment (start 113.94 95.19) (end 119.13 90) (width 0.8) (layer "B.Cu") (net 10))
 (segment (start 113.94 107) (end 113.94 95.19) (width 0.8) (layer "B.Cu") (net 10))
 (segment (start 115.9 110.04) (end 115.94 110) (width 0.8) (layer "B.Cu") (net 25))
 (segment (start 115.94 110) (end 115.94 95.69) (width 0.8) (layer "B.Cu") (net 25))
 (segment (start 113.44 110.04) (end 115.9 110.04) (width 0.8) (layer "B.Cu") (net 25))
 (segment (start 115.94 95.69) (end 119.13 92.5) (width 0.8) (layer "B.Cu") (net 25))
 (segment (start 115.86 112.58) (end 117.44 111) (width 0.8) (layer "B.Cu") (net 6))
 (segment (start 113.44 112.58) (end 115.86 112.58) (width 0.8) (layer "B.Cu") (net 6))
 (segment (start 117.44 111) (end 117.44 96.69) (width 0.8) (layer "B.Cu") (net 6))
 (segment (start 117.44 96.69) (end 119.13 95) (width 0.8) (layer "B.Cu") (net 6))
 (segment (start 116.865 115.075) (end 118.94 113) (width 0.8) (layer "B.Cu") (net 26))
 (segment (start 113.485 115.075) (end 116.865 115.075) (width 0.8) (layer "B.Cu") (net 26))
 (segment (start 113.44 115.12) (end 113.485 115.075) (width 0.8) (layer "B.Cu") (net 26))
 (segment (start 118.94 113) (end 118.94 98) (width 0.8) (layer "B.Cu") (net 26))
 (segment (start 158.44 97.4) (end 159.739511 98.699511) (width 0.8) (layer "B.Cu") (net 1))
 (segment (start 148.049511 122.199511) (end 145.75 119.9) (width 0.8) (layer "B.Cu") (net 1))
 (segment (start 138.13 122.19) (end 139.44 123.5) (width 0.8) (layer "B.Cu") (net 1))
 (segment (start 153.950489 122.199511) (end 148.049511 122.199511) (width 0.8) (layer "B.Cu") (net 1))
 (segment (start 159.739511 117.100489) (end 159.13 117.71) (width 0.8) (layer "B.Cu") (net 1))
 (segment (start 165.44 120.5) (end 162.260489 123.679511) (width 0.8) (layer "B.Cu") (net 1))
 (segment (start 159.739511 106.410489) (end 158.44 107.71) (width 0.8) (layer "B.Cu") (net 1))
 (segment (start 158.44 107.71) (end 159.739511 109.009511) (width 0.8) (layer "B.Cu") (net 1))
 (segment (start 138.13 119.9) (end 138.13 122.19) (width 0.8) (layer "B.Cu") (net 1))
 (segment (start 159.13 117.71) (end 158.44 117.71) (width 0.8) (layer "B.Cu") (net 1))
 (segment (start 159.749022 109) (end 159.739511 109.009511) (width 0.8) (layer "B.Cu") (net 1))
 (segment (start 165.44 109.015) (end 161.73 109.015) (width 0.8) (layer "B.Cu") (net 1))
 (segment (start 158.44 117.71) (end 153.950489 122.199511) (width 0.8) (layer "B.Cu") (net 1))
 (segment (start 159.745 111) (end 159.739511 110.994511) (width 0.8) (layer "B.Cu") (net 1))
 (segment (start 127.66 123.5) (end 126.44 122.28) (width 0.8) (layer "B.Cu") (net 1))
 (segment (start 162.260489 123.679511) (end 127.839511 123.679511) (width 0.8) (layer "B.Cu") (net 1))
 (segment (start 165.44 111.555) (end 165.44 120.5) (width 0.8) (layer "B.Cu") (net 1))
 (segment (start 161.73 109.015) (end 159.745 111) (width 0.8) (layer "B.Cu") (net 1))
 (segment (start 159.739511 98.699511) (end 159.739511 106.410489) (width 0.8) (layer "B.Cu") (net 1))
 (segment (start 159.739511 109.009511) (end 159.739511 117.100489) (width 0.8) (layer "B.Cu") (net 1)))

